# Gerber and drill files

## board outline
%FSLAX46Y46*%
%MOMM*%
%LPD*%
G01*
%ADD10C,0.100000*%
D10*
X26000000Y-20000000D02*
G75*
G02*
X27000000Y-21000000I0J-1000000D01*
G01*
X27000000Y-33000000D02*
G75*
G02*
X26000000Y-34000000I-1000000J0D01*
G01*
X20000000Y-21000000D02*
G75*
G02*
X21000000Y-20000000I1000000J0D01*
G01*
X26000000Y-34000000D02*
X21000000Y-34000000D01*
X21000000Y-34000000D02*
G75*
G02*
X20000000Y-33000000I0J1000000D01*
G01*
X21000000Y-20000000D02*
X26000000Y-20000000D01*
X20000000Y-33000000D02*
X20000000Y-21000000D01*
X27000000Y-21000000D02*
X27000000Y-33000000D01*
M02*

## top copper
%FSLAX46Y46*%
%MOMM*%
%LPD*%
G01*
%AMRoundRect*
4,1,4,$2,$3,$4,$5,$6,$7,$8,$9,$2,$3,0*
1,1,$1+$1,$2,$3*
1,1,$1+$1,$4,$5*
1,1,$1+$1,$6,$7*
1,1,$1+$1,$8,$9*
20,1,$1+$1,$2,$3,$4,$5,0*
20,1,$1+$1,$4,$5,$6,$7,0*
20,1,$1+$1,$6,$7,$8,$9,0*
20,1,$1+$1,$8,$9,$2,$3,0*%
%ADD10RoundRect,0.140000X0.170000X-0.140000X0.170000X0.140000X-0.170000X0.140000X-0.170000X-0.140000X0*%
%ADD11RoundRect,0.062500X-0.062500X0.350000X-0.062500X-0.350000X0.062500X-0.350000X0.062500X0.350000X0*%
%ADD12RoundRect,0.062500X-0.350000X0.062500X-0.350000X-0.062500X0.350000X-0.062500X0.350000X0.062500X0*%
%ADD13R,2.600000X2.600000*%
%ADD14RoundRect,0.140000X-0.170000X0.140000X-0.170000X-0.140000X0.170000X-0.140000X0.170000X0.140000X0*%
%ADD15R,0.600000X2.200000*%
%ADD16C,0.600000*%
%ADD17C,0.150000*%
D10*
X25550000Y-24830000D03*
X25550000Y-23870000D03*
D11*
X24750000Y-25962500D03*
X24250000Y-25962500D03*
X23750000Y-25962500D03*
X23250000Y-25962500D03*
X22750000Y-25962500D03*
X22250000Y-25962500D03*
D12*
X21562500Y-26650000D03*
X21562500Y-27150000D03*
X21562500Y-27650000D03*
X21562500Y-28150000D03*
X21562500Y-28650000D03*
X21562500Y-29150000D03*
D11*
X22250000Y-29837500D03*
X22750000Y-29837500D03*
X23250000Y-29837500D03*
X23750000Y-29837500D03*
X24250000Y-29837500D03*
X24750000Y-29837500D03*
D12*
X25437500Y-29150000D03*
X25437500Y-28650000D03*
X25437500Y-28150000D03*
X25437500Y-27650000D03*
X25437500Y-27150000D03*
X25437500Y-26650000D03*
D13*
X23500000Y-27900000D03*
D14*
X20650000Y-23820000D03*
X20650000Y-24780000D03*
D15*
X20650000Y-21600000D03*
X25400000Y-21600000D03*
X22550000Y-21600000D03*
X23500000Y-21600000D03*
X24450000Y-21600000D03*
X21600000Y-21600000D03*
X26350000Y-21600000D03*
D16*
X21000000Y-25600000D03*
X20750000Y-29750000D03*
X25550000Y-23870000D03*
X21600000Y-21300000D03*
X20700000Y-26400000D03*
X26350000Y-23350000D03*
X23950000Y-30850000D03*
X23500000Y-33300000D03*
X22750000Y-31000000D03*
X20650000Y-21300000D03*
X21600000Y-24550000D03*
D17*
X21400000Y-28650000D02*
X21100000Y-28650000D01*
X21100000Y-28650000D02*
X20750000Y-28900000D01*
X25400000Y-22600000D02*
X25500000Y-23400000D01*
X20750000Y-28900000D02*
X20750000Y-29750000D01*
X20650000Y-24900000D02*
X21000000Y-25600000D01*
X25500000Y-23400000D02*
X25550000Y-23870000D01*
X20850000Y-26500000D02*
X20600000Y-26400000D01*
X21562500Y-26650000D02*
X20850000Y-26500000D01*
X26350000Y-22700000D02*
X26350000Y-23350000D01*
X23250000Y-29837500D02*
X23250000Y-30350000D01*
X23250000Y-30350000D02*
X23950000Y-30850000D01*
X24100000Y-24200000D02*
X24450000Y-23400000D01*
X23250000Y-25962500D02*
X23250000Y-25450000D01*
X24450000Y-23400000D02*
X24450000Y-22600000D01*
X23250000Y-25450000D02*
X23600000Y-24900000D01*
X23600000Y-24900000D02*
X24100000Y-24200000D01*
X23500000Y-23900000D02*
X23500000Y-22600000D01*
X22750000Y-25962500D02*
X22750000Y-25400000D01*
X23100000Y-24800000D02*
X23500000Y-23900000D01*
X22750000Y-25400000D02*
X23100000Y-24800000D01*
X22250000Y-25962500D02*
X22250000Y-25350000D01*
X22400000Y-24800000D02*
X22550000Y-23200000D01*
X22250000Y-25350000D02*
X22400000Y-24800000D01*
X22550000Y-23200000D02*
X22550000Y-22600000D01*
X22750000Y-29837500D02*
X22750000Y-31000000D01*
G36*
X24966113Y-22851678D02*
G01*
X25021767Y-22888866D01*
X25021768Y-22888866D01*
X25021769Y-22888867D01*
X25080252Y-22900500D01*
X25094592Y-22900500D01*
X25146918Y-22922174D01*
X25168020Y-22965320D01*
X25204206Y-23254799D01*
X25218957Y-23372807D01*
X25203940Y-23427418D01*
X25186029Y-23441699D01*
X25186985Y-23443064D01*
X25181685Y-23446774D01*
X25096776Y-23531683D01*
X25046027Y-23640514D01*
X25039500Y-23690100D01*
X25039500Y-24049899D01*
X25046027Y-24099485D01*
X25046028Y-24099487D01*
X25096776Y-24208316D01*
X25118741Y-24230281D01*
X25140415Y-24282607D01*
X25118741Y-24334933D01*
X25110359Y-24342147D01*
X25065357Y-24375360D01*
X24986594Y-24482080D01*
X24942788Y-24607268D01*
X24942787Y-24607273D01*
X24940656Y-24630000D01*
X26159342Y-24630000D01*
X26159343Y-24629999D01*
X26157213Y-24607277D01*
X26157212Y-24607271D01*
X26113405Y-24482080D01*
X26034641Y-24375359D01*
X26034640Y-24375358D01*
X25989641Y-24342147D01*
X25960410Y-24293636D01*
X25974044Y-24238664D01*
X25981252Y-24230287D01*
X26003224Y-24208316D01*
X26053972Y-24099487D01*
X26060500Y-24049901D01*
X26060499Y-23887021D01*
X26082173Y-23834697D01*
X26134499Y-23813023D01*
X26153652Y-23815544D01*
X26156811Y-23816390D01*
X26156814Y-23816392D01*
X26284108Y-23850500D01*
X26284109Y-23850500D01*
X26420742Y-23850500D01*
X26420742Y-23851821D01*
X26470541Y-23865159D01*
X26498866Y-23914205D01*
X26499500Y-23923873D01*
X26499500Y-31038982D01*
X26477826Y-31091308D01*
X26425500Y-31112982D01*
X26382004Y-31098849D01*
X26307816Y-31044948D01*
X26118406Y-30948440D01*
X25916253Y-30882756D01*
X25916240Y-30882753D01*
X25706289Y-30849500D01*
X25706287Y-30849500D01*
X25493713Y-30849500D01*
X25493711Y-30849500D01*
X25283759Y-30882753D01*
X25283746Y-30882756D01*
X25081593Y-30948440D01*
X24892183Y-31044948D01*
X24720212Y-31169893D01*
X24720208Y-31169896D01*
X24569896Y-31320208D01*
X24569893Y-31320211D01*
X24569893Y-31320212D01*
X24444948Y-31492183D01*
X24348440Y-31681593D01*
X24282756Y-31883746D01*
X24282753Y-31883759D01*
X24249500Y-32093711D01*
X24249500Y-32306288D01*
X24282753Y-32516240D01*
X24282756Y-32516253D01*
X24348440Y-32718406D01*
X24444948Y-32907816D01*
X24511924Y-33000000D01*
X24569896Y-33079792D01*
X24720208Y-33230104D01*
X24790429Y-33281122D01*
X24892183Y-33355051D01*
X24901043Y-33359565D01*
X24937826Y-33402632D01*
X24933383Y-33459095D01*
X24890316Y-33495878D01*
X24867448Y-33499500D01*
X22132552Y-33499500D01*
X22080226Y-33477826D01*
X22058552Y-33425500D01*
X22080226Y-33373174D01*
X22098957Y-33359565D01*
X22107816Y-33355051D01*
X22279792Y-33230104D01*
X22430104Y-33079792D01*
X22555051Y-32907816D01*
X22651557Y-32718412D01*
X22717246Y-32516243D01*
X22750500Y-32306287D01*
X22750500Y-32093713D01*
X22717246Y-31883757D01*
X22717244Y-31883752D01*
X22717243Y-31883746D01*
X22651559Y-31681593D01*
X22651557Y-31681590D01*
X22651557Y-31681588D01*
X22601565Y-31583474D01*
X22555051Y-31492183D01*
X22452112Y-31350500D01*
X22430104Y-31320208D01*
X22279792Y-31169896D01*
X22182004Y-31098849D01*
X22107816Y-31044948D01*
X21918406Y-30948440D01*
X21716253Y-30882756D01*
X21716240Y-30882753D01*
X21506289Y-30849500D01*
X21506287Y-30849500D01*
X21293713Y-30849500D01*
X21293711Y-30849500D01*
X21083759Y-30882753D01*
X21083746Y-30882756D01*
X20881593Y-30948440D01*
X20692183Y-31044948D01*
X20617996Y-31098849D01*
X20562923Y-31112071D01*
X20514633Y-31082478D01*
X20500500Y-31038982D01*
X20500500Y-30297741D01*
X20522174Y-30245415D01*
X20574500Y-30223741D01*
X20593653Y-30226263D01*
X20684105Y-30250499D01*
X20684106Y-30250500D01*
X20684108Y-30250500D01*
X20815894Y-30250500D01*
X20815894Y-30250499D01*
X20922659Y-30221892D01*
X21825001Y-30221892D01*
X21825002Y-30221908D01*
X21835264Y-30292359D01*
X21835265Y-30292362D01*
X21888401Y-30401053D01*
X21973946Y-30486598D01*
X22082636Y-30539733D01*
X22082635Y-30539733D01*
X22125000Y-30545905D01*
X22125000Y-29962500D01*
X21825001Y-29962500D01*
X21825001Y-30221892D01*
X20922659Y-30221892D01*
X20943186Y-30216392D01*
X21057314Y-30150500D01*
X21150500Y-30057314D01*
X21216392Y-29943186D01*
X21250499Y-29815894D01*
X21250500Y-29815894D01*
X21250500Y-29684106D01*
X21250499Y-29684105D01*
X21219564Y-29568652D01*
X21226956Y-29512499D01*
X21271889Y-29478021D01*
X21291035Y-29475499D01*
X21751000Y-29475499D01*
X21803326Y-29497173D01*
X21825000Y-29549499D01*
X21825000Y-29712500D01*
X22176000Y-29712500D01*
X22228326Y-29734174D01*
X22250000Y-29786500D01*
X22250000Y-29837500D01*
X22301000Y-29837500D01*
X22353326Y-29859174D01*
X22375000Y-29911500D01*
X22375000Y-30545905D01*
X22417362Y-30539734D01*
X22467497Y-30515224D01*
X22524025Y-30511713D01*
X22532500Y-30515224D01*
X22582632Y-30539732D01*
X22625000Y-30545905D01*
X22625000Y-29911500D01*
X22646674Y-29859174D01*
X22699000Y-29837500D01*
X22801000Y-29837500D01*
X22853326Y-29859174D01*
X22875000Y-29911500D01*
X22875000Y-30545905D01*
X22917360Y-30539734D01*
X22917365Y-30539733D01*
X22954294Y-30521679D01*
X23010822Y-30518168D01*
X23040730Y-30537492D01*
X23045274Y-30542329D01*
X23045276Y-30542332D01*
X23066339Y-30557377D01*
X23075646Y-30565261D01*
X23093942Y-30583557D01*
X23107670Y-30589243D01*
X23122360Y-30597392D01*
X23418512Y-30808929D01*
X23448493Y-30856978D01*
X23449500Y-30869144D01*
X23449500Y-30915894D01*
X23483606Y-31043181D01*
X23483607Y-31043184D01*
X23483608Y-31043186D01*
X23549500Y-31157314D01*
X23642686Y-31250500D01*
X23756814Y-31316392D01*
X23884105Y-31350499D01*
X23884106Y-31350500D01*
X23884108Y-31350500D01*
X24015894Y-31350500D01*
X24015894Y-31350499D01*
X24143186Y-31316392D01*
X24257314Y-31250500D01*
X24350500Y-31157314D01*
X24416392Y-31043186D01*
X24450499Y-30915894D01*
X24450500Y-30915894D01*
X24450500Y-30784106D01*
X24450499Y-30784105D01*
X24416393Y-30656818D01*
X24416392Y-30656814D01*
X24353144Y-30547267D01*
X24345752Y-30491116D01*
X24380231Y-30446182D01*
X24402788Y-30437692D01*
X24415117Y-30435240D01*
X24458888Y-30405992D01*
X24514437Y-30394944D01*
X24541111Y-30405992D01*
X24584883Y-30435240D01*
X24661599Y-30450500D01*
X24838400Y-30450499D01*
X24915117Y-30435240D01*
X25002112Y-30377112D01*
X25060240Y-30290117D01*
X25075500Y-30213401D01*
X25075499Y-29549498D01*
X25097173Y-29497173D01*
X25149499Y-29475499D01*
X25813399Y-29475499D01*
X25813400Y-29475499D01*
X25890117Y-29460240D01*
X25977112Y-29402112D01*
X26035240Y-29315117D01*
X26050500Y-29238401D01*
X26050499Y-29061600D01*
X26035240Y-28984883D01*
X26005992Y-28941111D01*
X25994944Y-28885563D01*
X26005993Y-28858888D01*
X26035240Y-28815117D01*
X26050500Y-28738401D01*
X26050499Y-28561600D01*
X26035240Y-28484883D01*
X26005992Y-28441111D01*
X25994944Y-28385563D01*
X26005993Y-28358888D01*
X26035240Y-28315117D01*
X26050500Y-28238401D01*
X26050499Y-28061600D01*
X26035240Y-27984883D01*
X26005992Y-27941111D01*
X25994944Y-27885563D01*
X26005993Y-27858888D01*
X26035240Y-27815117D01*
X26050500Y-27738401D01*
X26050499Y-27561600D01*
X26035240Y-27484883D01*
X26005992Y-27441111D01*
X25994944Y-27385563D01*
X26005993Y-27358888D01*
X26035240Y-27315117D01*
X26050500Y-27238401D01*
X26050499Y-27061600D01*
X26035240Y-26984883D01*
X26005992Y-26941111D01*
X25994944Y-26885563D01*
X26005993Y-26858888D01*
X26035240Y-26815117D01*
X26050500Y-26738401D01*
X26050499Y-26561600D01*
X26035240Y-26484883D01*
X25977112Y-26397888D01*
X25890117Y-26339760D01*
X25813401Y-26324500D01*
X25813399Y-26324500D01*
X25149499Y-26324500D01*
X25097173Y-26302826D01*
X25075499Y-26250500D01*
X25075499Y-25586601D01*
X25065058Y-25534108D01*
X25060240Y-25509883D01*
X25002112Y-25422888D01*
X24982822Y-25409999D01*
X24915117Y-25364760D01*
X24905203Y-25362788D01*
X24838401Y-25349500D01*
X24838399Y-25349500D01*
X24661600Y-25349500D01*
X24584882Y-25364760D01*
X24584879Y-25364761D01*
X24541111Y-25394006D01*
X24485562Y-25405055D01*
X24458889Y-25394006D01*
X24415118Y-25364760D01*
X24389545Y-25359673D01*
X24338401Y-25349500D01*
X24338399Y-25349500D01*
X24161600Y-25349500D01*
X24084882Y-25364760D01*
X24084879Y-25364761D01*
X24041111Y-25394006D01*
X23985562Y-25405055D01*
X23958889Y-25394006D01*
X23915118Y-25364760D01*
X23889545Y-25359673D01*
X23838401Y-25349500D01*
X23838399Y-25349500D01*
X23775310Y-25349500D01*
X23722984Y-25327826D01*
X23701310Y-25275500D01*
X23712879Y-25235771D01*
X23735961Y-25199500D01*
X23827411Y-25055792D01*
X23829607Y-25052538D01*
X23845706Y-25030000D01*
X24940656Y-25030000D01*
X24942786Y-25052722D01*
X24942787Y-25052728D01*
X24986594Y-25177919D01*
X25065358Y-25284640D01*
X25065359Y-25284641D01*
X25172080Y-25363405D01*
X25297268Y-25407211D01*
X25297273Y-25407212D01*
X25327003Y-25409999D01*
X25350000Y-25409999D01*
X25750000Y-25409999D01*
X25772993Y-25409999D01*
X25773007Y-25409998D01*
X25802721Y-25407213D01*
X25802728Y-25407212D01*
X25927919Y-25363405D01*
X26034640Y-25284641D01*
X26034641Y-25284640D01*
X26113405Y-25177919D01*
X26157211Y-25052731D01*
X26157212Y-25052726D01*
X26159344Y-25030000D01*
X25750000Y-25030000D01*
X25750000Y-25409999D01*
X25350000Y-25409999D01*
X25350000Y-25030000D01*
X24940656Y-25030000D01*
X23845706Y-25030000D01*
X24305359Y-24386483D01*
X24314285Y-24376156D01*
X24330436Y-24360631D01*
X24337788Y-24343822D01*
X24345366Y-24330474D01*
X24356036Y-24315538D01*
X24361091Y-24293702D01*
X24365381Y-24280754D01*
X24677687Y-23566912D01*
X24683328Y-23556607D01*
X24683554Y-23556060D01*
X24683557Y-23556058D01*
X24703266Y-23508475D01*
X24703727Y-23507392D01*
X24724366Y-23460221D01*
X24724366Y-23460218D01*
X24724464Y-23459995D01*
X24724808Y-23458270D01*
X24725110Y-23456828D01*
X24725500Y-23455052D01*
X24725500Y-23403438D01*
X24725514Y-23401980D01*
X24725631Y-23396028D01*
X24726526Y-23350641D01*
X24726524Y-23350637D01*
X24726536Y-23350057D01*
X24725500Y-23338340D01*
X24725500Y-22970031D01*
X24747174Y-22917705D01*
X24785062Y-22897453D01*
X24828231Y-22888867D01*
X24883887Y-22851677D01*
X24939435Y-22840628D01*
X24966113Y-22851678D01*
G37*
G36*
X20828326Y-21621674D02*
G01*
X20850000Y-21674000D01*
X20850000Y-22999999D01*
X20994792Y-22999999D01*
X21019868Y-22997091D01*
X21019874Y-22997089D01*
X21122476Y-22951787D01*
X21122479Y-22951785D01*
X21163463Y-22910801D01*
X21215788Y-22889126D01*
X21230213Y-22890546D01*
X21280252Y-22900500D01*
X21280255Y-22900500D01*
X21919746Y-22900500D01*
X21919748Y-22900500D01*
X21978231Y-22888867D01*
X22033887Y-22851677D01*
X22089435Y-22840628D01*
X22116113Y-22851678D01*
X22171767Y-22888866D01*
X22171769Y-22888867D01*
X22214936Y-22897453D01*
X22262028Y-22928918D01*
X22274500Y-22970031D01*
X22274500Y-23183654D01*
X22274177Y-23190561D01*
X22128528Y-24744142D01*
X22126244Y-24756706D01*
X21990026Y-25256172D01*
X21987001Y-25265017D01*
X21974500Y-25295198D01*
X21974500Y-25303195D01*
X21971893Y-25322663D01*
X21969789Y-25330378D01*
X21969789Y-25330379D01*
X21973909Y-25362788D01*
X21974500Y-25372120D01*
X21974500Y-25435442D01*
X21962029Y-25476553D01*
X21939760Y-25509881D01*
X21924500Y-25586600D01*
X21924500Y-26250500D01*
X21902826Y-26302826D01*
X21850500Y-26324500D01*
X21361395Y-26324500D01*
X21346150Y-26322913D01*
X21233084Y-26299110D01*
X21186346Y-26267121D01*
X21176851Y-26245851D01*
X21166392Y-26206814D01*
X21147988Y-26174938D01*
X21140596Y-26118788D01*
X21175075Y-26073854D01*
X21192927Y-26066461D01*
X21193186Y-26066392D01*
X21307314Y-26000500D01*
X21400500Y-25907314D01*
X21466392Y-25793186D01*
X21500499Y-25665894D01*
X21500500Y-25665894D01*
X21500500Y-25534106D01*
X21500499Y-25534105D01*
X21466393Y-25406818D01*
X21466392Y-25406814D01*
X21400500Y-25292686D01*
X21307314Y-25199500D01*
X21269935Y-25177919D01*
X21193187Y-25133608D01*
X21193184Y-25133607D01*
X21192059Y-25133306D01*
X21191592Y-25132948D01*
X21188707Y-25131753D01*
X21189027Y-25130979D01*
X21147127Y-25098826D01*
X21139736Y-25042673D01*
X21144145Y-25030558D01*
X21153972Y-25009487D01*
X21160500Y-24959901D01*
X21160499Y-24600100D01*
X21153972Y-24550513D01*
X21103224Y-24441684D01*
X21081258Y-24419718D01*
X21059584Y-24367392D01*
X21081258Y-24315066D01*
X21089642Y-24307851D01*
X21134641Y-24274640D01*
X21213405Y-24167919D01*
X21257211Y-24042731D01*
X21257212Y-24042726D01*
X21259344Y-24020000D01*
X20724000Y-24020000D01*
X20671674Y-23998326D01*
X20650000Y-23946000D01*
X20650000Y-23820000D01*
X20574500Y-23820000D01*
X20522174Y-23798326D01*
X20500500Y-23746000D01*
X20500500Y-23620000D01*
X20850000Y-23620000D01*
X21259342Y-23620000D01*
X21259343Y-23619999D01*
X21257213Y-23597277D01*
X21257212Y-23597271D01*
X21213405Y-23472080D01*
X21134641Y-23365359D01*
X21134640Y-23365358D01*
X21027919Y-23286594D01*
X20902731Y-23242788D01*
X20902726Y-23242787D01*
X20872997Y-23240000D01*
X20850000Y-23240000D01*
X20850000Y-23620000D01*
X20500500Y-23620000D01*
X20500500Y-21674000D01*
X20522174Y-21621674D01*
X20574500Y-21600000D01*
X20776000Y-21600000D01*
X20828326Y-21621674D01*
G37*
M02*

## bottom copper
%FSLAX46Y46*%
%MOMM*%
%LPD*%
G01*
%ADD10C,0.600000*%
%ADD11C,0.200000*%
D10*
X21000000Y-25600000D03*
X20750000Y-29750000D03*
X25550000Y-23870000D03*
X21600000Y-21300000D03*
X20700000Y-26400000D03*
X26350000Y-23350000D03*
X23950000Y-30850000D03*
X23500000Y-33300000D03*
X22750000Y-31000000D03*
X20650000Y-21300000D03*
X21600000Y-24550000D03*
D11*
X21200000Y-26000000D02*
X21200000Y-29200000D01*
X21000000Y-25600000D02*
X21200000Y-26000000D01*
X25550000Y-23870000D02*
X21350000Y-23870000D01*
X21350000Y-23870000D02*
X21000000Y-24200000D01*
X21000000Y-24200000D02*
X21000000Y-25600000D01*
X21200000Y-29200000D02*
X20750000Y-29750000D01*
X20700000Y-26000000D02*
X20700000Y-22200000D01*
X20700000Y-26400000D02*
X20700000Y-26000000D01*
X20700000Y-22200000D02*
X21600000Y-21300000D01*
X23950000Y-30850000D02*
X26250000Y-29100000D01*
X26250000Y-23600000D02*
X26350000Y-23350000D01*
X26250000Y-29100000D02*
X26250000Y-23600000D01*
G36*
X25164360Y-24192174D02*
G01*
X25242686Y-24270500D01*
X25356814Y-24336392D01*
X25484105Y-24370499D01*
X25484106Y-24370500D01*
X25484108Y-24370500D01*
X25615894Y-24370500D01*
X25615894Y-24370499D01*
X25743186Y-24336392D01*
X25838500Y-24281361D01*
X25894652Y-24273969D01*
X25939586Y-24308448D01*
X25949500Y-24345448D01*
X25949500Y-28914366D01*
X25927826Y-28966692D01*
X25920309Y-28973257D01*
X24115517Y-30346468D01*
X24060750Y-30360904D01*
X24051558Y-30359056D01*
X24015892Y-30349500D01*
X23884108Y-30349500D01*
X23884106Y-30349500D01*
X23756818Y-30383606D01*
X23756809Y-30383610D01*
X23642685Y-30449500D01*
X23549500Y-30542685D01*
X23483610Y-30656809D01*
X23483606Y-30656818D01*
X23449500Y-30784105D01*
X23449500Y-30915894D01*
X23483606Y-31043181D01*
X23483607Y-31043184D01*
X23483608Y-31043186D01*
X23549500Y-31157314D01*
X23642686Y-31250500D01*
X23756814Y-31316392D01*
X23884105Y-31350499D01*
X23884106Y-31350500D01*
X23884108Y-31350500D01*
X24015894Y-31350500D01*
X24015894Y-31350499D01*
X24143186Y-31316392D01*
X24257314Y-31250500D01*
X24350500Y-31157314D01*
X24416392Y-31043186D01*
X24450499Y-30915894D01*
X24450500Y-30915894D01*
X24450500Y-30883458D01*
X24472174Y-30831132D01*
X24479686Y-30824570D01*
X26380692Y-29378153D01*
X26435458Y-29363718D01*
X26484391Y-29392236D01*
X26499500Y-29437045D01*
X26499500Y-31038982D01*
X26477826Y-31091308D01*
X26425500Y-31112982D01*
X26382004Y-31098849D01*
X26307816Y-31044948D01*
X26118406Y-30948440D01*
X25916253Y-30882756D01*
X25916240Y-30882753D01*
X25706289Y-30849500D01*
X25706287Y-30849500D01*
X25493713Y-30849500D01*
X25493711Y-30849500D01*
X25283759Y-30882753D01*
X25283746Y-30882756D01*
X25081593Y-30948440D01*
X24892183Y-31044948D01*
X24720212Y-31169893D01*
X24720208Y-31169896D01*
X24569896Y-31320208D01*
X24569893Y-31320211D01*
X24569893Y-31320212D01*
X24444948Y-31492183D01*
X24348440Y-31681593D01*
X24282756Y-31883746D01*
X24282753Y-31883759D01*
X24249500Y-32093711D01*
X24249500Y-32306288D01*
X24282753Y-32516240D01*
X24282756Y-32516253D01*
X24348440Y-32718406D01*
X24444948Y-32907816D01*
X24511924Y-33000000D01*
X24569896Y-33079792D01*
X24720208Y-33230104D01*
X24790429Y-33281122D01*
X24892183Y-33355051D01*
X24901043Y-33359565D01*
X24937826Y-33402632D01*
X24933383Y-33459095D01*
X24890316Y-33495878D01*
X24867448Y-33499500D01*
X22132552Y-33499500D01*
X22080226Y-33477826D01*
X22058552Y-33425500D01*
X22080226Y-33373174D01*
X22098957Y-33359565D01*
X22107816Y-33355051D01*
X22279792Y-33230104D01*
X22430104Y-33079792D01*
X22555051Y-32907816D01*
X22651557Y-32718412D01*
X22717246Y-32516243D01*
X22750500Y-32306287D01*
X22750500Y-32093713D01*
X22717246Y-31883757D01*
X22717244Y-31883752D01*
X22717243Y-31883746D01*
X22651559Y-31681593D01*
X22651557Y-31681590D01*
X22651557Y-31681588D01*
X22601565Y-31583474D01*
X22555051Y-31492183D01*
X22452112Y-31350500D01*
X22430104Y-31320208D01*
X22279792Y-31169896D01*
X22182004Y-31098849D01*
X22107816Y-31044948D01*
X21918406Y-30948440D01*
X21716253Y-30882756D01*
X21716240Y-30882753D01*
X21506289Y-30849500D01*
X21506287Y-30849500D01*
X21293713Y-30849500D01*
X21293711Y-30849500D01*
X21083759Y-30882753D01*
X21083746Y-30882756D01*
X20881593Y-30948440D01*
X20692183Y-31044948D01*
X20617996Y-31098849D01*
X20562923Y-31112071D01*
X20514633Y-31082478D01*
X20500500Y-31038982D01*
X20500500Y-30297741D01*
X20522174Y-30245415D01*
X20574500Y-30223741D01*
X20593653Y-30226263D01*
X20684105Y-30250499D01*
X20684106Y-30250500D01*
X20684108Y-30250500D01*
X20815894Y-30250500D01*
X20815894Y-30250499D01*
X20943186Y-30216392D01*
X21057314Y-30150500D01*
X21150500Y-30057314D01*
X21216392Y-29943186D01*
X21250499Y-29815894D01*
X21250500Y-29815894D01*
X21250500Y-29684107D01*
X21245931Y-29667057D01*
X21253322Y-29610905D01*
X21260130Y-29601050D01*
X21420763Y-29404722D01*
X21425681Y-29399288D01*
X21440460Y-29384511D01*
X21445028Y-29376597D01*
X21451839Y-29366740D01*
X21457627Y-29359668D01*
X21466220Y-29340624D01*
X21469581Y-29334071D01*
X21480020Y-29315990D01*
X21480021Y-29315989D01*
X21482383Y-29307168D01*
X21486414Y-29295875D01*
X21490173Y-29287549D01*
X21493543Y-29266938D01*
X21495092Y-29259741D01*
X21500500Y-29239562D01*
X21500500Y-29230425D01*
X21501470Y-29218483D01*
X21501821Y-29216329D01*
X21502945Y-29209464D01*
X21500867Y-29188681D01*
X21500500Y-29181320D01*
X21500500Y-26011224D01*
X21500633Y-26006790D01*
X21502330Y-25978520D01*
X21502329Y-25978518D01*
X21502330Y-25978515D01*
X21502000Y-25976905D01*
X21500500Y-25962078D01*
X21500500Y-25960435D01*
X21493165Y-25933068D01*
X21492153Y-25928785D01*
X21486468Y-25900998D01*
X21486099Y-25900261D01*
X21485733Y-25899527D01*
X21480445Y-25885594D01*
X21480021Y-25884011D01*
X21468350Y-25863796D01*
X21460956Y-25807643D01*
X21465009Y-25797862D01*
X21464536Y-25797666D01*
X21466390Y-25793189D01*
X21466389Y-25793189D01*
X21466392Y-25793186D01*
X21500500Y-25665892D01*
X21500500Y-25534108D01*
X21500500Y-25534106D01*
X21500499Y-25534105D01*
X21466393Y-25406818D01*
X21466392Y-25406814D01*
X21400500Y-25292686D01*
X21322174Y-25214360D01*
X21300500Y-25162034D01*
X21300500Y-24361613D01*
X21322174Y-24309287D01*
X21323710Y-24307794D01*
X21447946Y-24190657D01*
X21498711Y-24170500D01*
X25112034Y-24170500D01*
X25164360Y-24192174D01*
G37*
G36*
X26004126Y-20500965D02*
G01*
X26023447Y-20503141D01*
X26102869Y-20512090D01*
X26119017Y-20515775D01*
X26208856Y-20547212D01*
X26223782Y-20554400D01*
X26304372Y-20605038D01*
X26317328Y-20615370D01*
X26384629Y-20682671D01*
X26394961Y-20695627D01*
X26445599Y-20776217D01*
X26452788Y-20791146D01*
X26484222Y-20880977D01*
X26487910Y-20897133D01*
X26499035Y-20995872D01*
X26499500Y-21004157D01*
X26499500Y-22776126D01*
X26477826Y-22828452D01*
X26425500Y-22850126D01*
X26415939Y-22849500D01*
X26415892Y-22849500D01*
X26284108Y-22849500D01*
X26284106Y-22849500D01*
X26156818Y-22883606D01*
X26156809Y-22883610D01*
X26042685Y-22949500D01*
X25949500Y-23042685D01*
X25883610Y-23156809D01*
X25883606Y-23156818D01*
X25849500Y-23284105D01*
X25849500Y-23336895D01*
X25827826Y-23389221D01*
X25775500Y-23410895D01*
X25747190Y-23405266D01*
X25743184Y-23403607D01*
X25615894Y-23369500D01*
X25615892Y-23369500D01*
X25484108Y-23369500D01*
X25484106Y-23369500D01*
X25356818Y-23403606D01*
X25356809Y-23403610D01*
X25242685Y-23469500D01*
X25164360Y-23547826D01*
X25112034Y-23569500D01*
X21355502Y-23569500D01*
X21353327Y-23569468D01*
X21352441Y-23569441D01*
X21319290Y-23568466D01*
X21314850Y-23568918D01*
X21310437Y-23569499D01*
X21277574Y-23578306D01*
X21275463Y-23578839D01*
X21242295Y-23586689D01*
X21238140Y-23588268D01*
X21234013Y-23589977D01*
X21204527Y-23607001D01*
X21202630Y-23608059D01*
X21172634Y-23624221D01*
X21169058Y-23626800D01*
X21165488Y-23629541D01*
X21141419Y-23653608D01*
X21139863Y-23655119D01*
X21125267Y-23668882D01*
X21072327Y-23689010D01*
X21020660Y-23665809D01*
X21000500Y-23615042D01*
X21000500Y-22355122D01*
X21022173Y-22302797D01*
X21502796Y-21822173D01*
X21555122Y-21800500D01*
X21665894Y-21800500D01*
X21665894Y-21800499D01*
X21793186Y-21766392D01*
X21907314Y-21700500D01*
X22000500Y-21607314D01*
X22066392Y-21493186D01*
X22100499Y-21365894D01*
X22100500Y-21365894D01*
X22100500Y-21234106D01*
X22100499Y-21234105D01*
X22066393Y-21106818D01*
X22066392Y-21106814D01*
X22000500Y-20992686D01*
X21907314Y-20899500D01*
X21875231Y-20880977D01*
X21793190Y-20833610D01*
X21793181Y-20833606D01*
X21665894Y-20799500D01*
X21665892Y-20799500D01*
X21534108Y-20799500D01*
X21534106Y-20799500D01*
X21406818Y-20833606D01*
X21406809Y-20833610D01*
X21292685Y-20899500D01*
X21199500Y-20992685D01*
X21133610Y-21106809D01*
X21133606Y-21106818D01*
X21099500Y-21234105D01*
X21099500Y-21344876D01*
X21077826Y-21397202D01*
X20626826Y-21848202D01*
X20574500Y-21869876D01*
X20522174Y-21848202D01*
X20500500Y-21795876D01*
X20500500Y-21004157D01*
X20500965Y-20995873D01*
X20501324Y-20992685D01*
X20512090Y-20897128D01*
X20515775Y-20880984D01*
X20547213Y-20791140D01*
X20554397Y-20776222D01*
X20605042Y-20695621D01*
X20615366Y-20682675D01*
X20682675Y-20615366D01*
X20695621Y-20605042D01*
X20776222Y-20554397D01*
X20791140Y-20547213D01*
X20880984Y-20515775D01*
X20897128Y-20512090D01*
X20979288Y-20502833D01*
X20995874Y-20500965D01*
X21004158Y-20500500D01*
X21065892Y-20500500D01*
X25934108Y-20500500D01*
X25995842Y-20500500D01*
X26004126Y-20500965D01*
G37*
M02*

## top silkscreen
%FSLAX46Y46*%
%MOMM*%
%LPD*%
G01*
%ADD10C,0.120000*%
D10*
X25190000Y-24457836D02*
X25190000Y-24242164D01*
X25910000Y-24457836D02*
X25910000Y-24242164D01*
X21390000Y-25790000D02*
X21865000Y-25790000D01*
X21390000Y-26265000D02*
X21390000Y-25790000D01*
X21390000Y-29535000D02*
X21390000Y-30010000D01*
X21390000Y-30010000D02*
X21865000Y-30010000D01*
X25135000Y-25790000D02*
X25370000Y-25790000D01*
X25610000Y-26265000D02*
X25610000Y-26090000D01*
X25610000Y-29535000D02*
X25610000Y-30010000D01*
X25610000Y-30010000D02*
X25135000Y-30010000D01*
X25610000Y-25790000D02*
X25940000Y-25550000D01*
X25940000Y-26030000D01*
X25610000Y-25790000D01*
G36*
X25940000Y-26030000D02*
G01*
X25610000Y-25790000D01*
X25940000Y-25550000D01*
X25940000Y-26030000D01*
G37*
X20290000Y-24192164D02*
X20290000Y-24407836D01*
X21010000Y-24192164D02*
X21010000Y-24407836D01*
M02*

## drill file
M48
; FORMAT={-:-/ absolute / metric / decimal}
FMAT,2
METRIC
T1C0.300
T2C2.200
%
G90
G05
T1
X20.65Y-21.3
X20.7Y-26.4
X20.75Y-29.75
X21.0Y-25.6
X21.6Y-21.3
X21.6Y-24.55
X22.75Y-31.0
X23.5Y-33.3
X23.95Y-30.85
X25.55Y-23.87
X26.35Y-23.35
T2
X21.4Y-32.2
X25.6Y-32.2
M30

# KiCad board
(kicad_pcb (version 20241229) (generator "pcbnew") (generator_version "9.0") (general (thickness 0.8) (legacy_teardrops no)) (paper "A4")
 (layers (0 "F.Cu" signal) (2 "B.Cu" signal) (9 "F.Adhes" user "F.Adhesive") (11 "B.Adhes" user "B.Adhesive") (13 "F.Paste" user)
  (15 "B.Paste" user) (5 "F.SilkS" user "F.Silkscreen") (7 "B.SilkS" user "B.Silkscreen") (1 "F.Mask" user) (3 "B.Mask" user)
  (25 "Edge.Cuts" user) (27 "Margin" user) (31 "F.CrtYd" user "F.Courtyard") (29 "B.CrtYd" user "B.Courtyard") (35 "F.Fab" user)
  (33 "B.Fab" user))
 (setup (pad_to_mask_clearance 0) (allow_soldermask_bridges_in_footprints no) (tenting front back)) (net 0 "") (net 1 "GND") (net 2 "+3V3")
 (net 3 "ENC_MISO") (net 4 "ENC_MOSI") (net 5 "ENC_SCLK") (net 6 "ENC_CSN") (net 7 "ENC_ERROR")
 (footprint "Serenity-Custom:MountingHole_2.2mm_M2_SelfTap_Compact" (layer "F.Cu") (at 21.4 32.2)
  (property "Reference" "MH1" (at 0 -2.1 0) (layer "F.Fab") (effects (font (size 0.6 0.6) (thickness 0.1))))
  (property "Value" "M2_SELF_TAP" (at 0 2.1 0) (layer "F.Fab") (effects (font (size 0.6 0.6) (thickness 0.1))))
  (pad "" np_thru_hole circle (at 0 0) (size 2.2 2.2) (drill 2.2) (layers "*.Cu" "*.Mask")))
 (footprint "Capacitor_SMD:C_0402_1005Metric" (layer "F.Cu") (at 25.55 24.35 90)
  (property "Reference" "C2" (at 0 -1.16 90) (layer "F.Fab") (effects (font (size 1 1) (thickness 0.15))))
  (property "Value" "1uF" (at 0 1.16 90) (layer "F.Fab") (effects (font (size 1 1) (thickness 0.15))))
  (fp_line (start -0.107836 -0.36) (end 0.107836 -0.36) (stroke (width 0.12) (type solid)) (layer "F.SilkS"))
  (fp_line (start -0.107836 0.36) (end 0.107836 0.36) (stroke (width 0.12) (type solid)) (layer "F.SilkS"))
  (pad "1" smd roundrect (at -0.48 0 90) (size 0.56 0.62) (layers "F.Cu" "F.Mask" "F.Paste") (roundrect_rratio 0.25) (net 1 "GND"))
  (pad "2" smd roundrect (at 0.48 0 90) (size 0.56 0.62) (layers "F.Cu" "F.Mask" "F.Paste") (roundrect_rratio 0.25) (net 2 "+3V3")))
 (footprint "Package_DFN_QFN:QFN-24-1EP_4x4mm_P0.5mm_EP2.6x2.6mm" (layer "F.Cu") (at 23.5 27.9 -90)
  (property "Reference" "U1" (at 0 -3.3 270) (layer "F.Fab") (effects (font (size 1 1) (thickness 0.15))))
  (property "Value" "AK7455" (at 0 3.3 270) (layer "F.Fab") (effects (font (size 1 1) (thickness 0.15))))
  (fp_line (start -2.11 2.11) (end -2.11 1.635) (stroke (width 0.12) (type solid)) (layer "F.SilkS"))
  (fp_line (start -1.635 2.11) (end -2.11 2.11) (stroke (width 0.12) (type solid)) (layer "F.SilkS"))
  (fp_line (start 1.635 2.11) (end 2.11 2.11) (stroke (width 0.12) (type solid)) (layer "F.SilkS"))
  (fp_line (start 2.11 2.11) (end 2.11 1.635) (stroke (width 0.12) (type solid)) (layer "F.SilkS"))
  (fp_line (start -2.11 -1.635) (end -2.11 -1.87) (stroke (width 0.12) (type solid)) (layer "F.SilkS"))
  (fp_line (start -1.635 -2.11) (end -1.81 -2.11) (stroke (width 0.12) (type solid)) (layer "F.SilkS"))
  (fp_line (start 1.635 -2.11) (end 2.11 -2.11) (stroke (width 0.12) (type solid)) (layer "F.SilkS"))
  (fp_line (start 2.11 -2.11) (end 2.11 -1.635) (stroke (width 0.12) (type solid)) (layer "F.SilkS"))
  (fp_poly (pts (xy -2.11 -2.11) (xy -2.35 -2.44) (xy -1.87 -2.44)) (stroke (width 0.12) (type solid)) (fill yes) (layer "F.SilkS"))
  (pad "" smd roundrect (at -0.65 -0.65 270) (size 1.05 1.05) (layers "F.Paste") (roundrect_rratio 0.238095))
  (pad "" smd roundrect (at -0.65 0.65 270) (size 1.05 1.05) (layers "F.Paste") (roundrect_rratio 0.238095))
  (pad "" smd roundrect (at 0.65 -0.65 270) (size 1.05 1.05) (layers "F.Paste") (roundrect_rratio 0.238095))
  (pad "" smd roundrect (at 0.65 0.65 270) (size 1.05 1.05) (layers "F.Paste") (roundrect_rratio 0.238095))
  (pad "1" smd roundrect (at -1.9375 -1.25 270) (size 0.825 0.25) (layers "F.Cu" "F.Mask" "F.Paste") (roundrect_rratio 0.25))
  (pad "2" smd roundrect (at -1.9375 -0.75 270) (size 0.825 0.25) (layers "F.Cu" "F.Mask" "F.Paste") (roundrect_rratio 0.25))
  (pad "3" smd roundrect (at -1.9375 -0.25 270) (size 0.825 0.25) (layers "F.Cu" "F.Mask" "F.Paste") (roundrect_rratio 0.25))
  (pad "4" smd roundrect (at -1.9375 0.25 270) (size 0.825 0.25) (layers "F.Cu" "F.Mask" "F.Paste") (roundrect_rratio 0.25)
   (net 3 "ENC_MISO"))
  (pad "5" smd roundrect (at -1.9375 0.75 270) (size 0.825 0.25) (layers "F.Cu" "F.Mask" "F.Paste") (roundrect_rratio 0.25)
   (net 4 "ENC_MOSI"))
  (pad "6" smd roundrect (at -1.9375 1.25 270) (size 0.825 0.25) (layers "F.Cu" "F.Mask" "F.Paste") (roundrect_rratio 0.25)
   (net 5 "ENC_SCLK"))
  (pad "7" smd roundrect (at -1.25 1.9375 270) (size 0.25 0.825) (layers "F.Cu" "F.Mask" "F.Paste") (roundrect_rratio 0.25)
   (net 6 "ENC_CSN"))
  (pad "8" smd roundrect (at -0.75 1.9375 270) (size 0.25 0.825) (layers "F.Cu" "F.Mask" "F.Paste") (roundrect_rratio 0.25))
  (pad "9" smd roundrect (at -0.25 1.9375 270) (size 0.25 0.825) (layers "F.Cu" "F.Mask" "F.Paste") (roundrect_rratio 0.25))
  (pad "10" smd roundrect (at 0.25 1.9375 270) (size 0.25 0.825) (layers "F.Cu" "F.Mask" "F.Paste") (roundrect_rratio 0.25))
  (pad "11" smd roundrect (at 0.75 1.9375 270) (size 0.25 0.825) (layers "F.Cu" "F.Mask" "F.Paste") (roundrect_rratio 0.25) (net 2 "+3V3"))
  (pad "12" smd roundrect (at 1.25 1.9375 270) (size 0.25 0.825) (layers "F.Cu" "F.Mask" "F.Paste") (roundrect_rratio 0.25))
  (pad "13" smd roundrect (at 1.9375 1.25 270) (size 0.825 0.25) (layers "F.Cu" "F.Mask" "F.Paste") (roundrect_rratio 0.25) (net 1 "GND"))
  (pad "14" smd roundrect (at 1.9375 0.75 270) (size 0.825 0.25) (layers "F.Cu" "F.Mask" "F.Paste") (roundrect_rratio 0.25) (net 1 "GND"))
  (pad "15" smd roundrect (at 1.9375 0.25 270) (size 0.825 0.25) (layers "F.Cu" "F.Mask" "F.Paste") (roundrect_rratio 0.25)
   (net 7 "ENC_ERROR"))
  (pad "16" smd roundrect (at 1.9375 -0.25 270) (size 0.825 0.25) (layers "F.Cu" "F.Mask" "F.Paste") (roundrect_rratio 0.25))
  (pad "17" smd roundrect (at 1.9375 -0.75 270) (size 0.825 0.25) (layers "F.Cu" "F.Mask" "F.Paste") (roundrect_rratio 0.25))
  (pad "18" smd roundrect (at 1.9375 -1.25 270) (size 0.825 0.25) (layers "F.Cu" "F.Mask" "F.Paste") (roundrect_rratio 0.25))
  (pad "19" smd roundrect (at 1.25 -1.9375 270) (size 0.25 0.825) (layers "F.Cu" "F.Mask" "F.Paste") (roundrect_rratio 0.25))
  (pad "20" smd roundrect (at 0.75 -1.9375 270) (size 0.25 0.825) (layers "F.Cu" "F.Mask" "F.Paste") (roundrect_rratio 0.25))
  (pad "21" smd roundrect (at 0.25 -1.9375 270) (size 0.25 0.825) (layers "F.Cu" "F.Mask" "F.Paste") (roundrect_rratio 0.25))
  (pad "22" smd roundrect (at -0.25 -1.9375 270) (size 0.25 0.825) (layers "F.Cu" "F.Mask" "F.Paste") (roundrect_rratio 0.25))
  (pad "23" smd roundrect (at -0.75 -1.9375 270) (size 0.25 0.825) (layers "F.Cu" "F.Mask" "F.Paste") (roundrect_rratio 0.25))
  (pad "24" smd roundrect (at -1.25 -1.9375 270) (size 0.25 0.825) (layers "F.Cu" "F.Mask" "F.Paste") (roundrect_rratio 0.25))
  (pad "25" smd rect (at 0 0 270) (size 2.6 2.6) (layers "F.Cu" "F.Mask") (zone_connect 2)))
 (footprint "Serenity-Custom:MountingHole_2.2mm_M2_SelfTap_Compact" (layer "F.Cu") (at 25.6 32.2)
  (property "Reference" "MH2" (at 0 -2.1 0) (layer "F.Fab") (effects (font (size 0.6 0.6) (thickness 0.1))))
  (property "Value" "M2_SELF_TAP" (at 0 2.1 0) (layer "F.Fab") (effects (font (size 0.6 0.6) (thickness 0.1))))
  (pad "" np_thru_hole circle (at 0 0) (size 2.2 2.2) (drill 2.2) (layers "*.Cu" "*.Mask")))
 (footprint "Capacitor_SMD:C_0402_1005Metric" (layer "F.Cu") (at 20.65 24.3 -90)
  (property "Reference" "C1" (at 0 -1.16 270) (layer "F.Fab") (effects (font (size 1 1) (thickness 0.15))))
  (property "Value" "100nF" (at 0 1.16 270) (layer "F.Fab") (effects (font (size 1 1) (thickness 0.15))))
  (fp_line (start -0.107836 0.36) (end 0.107836 0.36) (stroke (width 0.12) (type solid)) (layer "F.SilkS"))
  (fp_line (start -0.107836 -0.36) (end 0.107836 -0.36) (stroke (width 0.12) (type solid)) (layer "F.SilkS"))
  (pad "1" smd roundrect (at -0.48 0 270) (size 0.56 0.62) (layers "F.Cu" "F.Mask" "F.Paste") (roundrect_rratio 0.25) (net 1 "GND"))
  (pad "2" smd roundrect (at 0.48 0 270) (size 0.56 0.62) (layers "F.Cu" "F.Mask" "F.Paste") (roundrect_rratio 0.25) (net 2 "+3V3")))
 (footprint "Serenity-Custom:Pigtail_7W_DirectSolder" (layer "F.Cu") (at 23.5 21.6)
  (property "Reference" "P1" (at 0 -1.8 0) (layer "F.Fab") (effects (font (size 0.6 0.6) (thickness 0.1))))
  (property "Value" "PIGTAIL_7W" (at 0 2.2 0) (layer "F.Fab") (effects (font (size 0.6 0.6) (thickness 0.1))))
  (pad "1" smd rect (at -2.85 0) (size 0.6 2.2) (layers "F.Cu" "F.Mask" "F.Paste") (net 1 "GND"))
  (pad "2" smd rect (at 1.9 0) (size 0.6 2.2) (layers "F.Cu" "F.Mask" "F.Paste") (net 2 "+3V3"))
  (pad "3" smd rect (at -0.95 0) (size 0.6 2.2) (layers "F.Cu" "F.Mask" "F.Paste") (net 5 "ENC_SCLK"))
  (pad "4" smd rect (at 0 0) (size 0.6 2.2) (layers "F.Cu" "F.Mask" "F.Paste") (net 4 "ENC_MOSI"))
  (pad "5" smd rect (at 0.95 0) (size 0.6 2.2) (layers "F.Cu" "F.Mask" "F.Paste") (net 3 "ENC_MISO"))
  (pad "6" smd rect (at -1.9 0) (size 0.6 2.2) (layers "F.Cu" "F.Mask" "F.Paste") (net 6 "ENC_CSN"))
  (pad "7" smd rect (at 2.85 0) (size 0.6 2.2) (layers "F.Cu" "F.Mask" "F.Paste") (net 7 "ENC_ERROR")))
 (gr_arc (start 26 20) (mid 26.707107 20.292893) (end 27 21) (stroke (width 0.1) (type solid)) (layer "Edge.Cuts"))
 (gr_arc (start 27 33) (mid 26.707107 33.707107) (end 26 34) (stroke (width 0.1) (type solid)) (layer "Edge.Cuts"))
 (gr_arc (start 20 21) (mid 20.292893 20.292893) (end 21 20) (stroke (width 0.1) (type solid)) (layer "Edge.Cuts"))
 (gr_line (start 26 34) (end 21 34) (stroke (width 0.1) (type solid)) (layer "Edge.Cuts"))
 (gr_arc (start 21 34) (mid 20.292893 33.707107) (end 20 33) (stroke (width 0.1) (type solid)) (layer "Edge.Cuts"))
 (gr_line (start 21 20) (end 26 20) (stroke (width 0.1) (type solid)) (layer "Edge.Cuts"))
 (gr_line (start 20 33) (end 20 21) (stroke (width 0.1) (type solid)) (layer "Edge.Cuts"))
 (gr_line (start 27 21) (end 27 33) (stroke (width 0.1) (type solid)) (layer "Edge.Cuts"))
 (segment (start 21.4 28.65) (end 21.1 28.65) (width 0.15) (layer "F.Cu") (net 2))
 (segment (start 21.1 28.65) (end 20.75 28.9) (width 0.15) (layer "F.Cu") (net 2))
 (segment (start 25.4 22.6) (end 25.5 23.4) (width 0.15) (layer "F.Cu") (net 2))
 (segment (start 20.75 28.9) (end 20.75 29.75) (width 0.15) (layer "F.Cu") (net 2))
 (segment (start 20.65 24.9) (end 21 25.6) (width 0.15) (layer "F.Cu") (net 2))
 (segment (start 25.5 23.4) (end 25.55 23.87) (width 0.15) (layer "F.Cu") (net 2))
 (via (at 21 25.6) (size 0.6) (drill 0.3) (layers "F.Cu" "B.Cu") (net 2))
 (via (at 20.75 29.75) (size 0.6) (drill 0.3) (layers "F.Cu" "B.Cu") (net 2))
 (via (at 25.55 23.87) (size 0.6) (drill 0.3) (layers "F.Cu" "B.Cu") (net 2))
 (segment (start 21.2 26) (end 21.2 29.2) (width 0.2) (layer "B.Cu") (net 2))
 (segment (start 21 25.6) (end 21.2 26) (width 0.2) (layer "B.Cu") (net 2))
 (segment (start 25.55 23.87) (end 21.35 23.87) (width 0.2) (layer "B.Cu") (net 2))
 (segment (start 21.35 23.87) (end 21 24.2) (width 0.2) (layer "B.Cu") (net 2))
 (segment (start 21 24.2) (end 21 25.6) (width 0.2) (layer "B.Cu") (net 2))
 (segment (start 21.2 29.2) (end 20.75 29.75) (width 0.2) (layer "B.Cu") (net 2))
 (segment (start 20.85 26.5) (end 20.6 26.4) (width 0.15) (layer "F.Cu") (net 6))
 (segment (start 21.5625 26.65) (end 20.85 26.5) (width 0.15) (layer "F.Cu") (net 6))
 (via (at 21.6 21.3) (size 0.6) (drill 0.3) (layers "F.Cu" "B.Cu") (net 6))
 (via (at 20.7 26.4) (size 0.6) (drill 0.3) (layers "F.Cu" "B.Cu") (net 6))
 (segment (start 20.7 26) (end 20.7 22.2) (width 0.2) (layer "B.Cu") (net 6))
 (segment (start 20.7 26.4) (end 20.7 26) (width 0.2) (layer "B.Cu") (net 6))
 (segment (start 20.7 22.2) (end 21.6 21.3) (width 0.2) (layer "B.Cu") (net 6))
 (segment (start 26.35 22.7) (end 26.35 23.35) (width 0.15) (layer "F.Cu") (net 7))
 (segment (start 23.25 29.8375) (end 23.25 30.35) (width 0.15) (layer "F.Cu") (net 7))
 (segment (start 23.25 30.35) (end 23.95 30.85) (width 0.15) (layer "F.Cu") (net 7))
 (via (at 26.35 23.35) (size 0.6) (drill 0.3) (layers "F.Cu" "B.Cu") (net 7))
 (via (at 23.95 30.85) (size 0.6) (drill 0.3) (layers "F.Cu" "B.Cu") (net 7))
 (segment (start 23.95 30.85) (end 26.25 29.1) (width 0.2) (layer "B.Cu") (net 7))
 (segment (start 26.25 23.6) (end 26.35 23.35) (width 0.2) (layer "B.Cu") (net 7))
 (segment (start 26.25 29.1) (end 26.25 23.6) (width 0.2) (layer "B.Cu") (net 7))
 (segment (start 24.1 24.2) (end 24.45 23.4) (width 0.15) (layer "F.Cu") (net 3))
 (segment (start 23.25 25.9625) (end 23.25 25.45) (width 0.15) (layer "F.Cu") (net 3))
 (segment (start 24.45 23.4) (end 24.45 22.6) (width 0.15) (layer "F.Cu") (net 3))
 (segment (start 23.25 25.45) (end 23.6 24.9) (width 0.15) (layer "F.Cu") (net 3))
 (segment (start 23.6 24.9) (end 24.1 24.2) (width 0.15) (layer "F.Cu") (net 3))
 (segment (start 23.5 23.9) (end 23.5 22.6) (width 0.15) (layer "F.Cu") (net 4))
 (segment (start 22.75 25.9625) (end 22.75 25.4) (width 0.15) (layer "F.Cu") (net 4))
 (segment (start 23.1 24.8) (end 23.5 23.9) (width 0.15) (layer "F.Cu") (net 4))
 (segment (start 22.75 25.4) (end 23.1 24.8) (width 0.15) (layer "F.Cu") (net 4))
 (segment (start 22.25 25.9625) (end 22.25 25.35) (width 0.15) (layer "F.Cu") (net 5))
 (segment (start 22.4 24.8) (end 22.55 23.2) (width 0.15) (layer "F.Cu") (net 5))
 (segment (start 22.25 25.35) (end 22.4 24.8) (width 0.15) (layer "F.Cu") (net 5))
 (segment (start 22.55 23.2) (end 22.55 22.6) (width 0.15) (layer "F.Cu") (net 5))
 (segment (start 22.75 29.8375) (end 22.75 31) (width 0.15) (layer "F.Cu") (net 1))
 (via (at 23.5 33.3) (size 0.6) (drill 0.3) (layers "F.Cu" "B.Cu") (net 1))
 (via (at 22.75 31) (size 0.6) (drill 0.3) (layers "F.Cu" "B.Cu") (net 1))
 (via (at 20.65 21.3) (size 0.6) (drill 0.3) (layers "F.Cu" "B.Cu") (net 1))
 (via (at 21.6 24.55) (size 0.6) (drill 0.3) (layers "F.Cu" "B.Cu") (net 1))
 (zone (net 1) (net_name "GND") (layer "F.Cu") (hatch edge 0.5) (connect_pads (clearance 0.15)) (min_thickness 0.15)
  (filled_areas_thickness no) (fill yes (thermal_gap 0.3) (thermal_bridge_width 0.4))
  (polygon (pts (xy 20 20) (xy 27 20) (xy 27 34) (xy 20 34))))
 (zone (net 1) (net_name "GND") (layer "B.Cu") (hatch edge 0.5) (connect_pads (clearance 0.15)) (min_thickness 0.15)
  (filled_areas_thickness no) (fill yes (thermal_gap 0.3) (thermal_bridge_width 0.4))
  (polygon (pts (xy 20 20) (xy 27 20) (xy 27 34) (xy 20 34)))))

